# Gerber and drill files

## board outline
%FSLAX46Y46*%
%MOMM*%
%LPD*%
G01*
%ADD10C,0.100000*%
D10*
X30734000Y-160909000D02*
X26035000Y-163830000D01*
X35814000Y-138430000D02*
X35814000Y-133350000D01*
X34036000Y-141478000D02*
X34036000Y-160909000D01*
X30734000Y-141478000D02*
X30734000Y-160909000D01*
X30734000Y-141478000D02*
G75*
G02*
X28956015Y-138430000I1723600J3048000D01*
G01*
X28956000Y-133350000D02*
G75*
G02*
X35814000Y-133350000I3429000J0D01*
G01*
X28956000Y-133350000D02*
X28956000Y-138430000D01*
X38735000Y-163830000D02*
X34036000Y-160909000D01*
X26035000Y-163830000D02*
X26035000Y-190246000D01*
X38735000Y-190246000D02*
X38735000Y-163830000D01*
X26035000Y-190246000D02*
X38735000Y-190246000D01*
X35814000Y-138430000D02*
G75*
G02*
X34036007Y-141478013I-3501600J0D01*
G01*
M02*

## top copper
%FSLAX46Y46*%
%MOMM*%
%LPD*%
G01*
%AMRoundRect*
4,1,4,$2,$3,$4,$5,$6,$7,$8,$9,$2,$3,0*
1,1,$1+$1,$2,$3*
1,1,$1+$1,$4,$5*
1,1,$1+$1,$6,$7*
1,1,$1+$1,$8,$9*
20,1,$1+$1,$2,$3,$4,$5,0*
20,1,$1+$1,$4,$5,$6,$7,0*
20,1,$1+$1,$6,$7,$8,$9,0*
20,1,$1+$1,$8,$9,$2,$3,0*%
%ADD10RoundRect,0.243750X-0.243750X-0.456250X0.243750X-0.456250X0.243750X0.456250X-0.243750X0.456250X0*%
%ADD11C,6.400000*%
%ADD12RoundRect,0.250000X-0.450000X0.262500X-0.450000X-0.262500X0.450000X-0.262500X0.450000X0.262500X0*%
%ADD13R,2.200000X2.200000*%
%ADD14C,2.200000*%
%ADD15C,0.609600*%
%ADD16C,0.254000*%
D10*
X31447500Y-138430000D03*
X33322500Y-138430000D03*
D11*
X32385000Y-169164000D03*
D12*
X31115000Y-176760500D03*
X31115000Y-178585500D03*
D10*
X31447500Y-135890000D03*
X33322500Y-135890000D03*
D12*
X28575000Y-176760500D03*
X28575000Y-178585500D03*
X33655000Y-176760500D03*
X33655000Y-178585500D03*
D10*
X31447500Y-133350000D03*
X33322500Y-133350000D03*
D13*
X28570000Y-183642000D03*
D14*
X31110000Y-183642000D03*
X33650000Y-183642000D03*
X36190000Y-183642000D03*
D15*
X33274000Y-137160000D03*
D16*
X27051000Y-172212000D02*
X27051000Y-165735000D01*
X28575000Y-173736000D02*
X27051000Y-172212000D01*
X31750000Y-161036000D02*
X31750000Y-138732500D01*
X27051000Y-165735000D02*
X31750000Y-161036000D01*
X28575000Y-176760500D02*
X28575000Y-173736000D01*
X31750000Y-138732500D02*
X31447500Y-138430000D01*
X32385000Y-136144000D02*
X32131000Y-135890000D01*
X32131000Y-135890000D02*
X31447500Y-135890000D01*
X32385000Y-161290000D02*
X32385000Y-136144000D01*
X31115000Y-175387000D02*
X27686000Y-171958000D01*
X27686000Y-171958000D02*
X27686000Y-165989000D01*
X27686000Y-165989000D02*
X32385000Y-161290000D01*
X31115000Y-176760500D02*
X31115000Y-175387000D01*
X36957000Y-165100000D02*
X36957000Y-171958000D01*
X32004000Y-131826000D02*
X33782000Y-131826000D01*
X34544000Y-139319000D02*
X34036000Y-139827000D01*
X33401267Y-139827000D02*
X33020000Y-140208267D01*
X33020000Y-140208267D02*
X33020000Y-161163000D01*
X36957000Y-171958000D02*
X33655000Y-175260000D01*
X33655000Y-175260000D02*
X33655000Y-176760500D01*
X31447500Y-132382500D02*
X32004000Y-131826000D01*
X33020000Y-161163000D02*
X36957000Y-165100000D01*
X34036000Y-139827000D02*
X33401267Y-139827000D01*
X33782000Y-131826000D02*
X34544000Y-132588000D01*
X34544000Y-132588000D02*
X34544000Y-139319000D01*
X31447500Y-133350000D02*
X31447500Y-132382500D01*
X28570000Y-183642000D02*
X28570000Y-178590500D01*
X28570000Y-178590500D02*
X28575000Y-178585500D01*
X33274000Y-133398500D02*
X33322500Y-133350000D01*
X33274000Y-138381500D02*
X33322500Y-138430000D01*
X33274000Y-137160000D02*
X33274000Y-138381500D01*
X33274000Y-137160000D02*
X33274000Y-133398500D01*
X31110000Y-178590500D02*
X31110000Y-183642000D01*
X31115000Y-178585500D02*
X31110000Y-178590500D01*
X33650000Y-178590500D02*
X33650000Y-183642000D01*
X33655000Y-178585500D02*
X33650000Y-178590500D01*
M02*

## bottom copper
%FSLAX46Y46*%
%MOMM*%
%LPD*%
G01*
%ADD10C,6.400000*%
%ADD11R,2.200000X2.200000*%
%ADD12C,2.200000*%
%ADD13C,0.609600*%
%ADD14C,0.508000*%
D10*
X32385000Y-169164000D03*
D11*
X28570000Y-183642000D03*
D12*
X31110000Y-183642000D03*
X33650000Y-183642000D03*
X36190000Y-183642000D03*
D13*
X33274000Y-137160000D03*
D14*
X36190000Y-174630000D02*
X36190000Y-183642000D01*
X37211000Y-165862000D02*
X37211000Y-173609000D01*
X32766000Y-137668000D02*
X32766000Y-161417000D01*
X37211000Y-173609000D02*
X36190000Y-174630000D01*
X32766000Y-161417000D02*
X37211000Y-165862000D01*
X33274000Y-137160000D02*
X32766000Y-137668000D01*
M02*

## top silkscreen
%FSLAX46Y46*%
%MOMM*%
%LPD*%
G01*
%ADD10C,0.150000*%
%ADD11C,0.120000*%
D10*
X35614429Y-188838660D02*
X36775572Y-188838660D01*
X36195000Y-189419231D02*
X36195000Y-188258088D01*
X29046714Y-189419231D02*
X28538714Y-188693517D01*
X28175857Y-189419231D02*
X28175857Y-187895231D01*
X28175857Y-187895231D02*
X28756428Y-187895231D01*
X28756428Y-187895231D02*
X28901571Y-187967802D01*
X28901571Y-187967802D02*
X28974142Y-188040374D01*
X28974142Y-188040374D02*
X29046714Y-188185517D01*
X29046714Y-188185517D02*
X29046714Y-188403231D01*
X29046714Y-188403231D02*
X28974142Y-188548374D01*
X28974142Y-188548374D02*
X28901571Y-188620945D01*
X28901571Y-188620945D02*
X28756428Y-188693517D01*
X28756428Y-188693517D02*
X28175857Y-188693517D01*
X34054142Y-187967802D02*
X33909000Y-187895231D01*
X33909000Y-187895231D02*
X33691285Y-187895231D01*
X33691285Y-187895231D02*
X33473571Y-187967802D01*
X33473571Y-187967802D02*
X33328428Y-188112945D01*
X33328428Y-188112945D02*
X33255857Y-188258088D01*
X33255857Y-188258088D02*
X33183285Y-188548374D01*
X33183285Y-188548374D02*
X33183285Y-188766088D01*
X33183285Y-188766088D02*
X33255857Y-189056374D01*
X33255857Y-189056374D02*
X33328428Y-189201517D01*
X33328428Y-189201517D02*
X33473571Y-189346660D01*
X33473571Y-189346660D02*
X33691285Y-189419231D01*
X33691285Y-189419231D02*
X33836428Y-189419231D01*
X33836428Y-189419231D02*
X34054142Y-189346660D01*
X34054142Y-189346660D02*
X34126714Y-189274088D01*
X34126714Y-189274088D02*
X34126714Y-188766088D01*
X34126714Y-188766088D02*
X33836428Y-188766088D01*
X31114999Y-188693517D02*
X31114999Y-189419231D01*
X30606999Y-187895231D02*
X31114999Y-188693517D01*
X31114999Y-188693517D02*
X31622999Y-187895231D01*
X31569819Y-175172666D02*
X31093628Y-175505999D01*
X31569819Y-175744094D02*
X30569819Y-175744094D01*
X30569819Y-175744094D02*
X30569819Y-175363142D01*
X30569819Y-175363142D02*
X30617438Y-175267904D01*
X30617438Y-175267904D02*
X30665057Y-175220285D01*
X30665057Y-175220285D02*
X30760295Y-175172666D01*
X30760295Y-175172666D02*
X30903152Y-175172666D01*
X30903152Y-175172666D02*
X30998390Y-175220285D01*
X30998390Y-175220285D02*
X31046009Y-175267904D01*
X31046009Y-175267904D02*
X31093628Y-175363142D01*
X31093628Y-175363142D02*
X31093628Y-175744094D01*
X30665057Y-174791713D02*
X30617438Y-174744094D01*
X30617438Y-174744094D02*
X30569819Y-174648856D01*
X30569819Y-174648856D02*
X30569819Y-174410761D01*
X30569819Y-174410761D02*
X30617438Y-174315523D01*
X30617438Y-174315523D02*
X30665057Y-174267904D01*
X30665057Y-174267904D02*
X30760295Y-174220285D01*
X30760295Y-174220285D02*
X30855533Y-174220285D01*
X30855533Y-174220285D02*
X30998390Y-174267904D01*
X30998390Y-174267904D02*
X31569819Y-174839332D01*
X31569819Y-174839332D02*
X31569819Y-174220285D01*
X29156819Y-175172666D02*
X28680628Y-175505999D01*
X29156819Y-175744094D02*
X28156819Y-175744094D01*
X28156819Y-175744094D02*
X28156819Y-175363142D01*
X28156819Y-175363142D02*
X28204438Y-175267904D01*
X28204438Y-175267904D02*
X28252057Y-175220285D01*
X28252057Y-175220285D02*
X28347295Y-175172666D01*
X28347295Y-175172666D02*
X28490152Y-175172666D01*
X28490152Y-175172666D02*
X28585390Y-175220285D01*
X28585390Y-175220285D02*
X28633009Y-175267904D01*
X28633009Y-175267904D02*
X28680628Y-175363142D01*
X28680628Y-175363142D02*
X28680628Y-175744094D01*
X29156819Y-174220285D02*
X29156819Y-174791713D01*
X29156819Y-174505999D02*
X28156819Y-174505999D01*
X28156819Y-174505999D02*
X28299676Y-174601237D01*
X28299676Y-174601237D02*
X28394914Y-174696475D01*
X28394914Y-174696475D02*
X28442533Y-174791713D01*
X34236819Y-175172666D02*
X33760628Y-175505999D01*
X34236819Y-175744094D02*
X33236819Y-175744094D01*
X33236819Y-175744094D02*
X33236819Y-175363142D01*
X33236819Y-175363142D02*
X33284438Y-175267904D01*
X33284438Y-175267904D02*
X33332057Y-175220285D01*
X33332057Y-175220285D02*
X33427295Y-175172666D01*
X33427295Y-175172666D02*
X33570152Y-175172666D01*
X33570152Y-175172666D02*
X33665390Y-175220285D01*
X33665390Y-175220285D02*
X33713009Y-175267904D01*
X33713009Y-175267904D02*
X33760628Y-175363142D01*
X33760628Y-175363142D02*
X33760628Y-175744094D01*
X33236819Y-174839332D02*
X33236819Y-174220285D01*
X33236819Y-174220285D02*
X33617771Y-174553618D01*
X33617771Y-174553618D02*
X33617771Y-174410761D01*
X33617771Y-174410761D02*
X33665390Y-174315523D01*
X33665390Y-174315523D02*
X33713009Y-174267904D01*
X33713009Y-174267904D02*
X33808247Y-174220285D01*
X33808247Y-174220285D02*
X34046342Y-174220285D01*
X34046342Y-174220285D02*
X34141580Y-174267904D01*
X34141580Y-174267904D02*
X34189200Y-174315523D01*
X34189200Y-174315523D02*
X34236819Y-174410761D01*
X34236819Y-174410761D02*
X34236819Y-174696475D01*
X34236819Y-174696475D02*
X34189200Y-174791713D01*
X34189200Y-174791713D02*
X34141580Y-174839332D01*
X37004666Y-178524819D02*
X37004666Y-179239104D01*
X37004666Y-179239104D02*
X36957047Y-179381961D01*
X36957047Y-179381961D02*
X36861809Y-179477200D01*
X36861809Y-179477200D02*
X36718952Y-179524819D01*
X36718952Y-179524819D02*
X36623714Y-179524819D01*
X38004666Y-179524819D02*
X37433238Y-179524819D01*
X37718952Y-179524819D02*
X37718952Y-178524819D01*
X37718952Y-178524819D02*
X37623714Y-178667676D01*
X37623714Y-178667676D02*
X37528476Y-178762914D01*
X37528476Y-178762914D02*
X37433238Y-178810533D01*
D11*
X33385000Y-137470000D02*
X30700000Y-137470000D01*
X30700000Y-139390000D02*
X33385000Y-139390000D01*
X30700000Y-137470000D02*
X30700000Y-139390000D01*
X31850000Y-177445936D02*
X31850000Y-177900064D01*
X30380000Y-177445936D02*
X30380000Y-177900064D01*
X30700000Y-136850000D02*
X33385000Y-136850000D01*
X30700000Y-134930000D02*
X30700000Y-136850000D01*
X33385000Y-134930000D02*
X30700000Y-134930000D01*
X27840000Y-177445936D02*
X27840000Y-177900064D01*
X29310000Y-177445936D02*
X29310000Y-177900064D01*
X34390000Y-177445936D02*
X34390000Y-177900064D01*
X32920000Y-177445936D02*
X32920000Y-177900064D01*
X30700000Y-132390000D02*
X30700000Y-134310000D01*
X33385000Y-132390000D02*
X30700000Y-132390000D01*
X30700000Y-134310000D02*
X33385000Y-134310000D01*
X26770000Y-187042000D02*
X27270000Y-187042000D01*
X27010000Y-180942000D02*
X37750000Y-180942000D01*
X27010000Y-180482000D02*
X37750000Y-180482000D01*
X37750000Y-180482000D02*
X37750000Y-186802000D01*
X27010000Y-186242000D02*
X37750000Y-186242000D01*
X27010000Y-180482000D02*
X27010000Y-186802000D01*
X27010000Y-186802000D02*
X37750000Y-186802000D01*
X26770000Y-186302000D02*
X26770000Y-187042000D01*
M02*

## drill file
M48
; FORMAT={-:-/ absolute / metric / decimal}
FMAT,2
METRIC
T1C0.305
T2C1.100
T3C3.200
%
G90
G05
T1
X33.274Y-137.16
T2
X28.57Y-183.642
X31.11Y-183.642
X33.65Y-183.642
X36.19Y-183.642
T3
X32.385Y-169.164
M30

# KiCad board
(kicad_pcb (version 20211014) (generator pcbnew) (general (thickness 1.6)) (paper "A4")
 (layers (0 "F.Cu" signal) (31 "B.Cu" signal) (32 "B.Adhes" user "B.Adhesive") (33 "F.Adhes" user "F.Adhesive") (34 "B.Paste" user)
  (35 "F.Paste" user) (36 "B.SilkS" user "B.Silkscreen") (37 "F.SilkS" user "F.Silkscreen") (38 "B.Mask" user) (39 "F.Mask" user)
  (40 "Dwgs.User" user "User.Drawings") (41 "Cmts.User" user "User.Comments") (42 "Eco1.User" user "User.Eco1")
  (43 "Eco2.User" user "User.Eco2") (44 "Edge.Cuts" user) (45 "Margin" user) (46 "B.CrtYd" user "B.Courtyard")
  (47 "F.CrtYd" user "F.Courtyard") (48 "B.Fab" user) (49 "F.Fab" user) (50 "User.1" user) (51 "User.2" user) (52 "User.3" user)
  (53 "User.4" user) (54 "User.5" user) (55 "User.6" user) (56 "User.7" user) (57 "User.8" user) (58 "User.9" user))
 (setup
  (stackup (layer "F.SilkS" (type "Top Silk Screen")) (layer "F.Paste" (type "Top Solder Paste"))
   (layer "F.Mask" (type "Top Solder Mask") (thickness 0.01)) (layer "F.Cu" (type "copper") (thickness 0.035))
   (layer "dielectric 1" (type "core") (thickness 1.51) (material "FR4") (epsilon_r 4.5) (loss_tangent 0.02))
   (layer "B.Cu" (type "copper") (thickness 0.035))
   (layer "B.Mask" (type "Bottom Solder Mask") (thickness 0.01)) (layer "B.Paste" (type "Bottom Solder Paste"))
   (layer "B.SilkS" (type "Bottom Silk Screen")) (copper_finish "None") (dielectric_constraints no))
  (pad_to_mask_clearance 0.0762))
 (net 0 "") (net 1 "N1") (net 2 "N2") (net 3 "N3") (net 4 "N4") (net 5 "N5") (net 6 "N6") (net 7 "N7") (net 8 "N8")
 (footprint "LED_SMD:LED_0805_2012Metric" (layer "F.Cu") (at 32.385 138.43)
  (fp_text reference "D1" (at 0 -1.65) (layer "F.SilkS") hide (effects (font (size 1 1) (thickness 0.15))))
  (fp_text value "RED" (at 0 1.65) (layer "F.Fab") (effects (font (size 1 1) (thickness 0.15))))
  (fp_line (start 1 -0.96) (end -1.685 -0.96) (layer "F.SilkS") (width 0.12))
  (fp_line (start -1.685 0.96) (end 1 0.96) (layer "F.SilkS") (width 0.12))
  (fp_line (start -1.685 -0.96) (end -1.685 0.96) (layer "F.SilkS") (width 0.12))
  (pad "1" smd roundrect (at -0.9375 0) (size 0.975 1.4) (layers "F.Cu" "F.Paste" "F.Mask") (roundrect_rratio 0.25) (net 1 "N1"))
  (pad "2" smd roundrect (at 0.9375 0) (size 0.975 1.4) (layers "F.Cu" "F.Paste" "F.Mask") (roundrect_rratio 0.25) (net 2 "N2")))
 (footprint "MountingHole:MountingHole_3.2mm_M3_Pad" (layer "F.Cu") (at 32.385 169.164) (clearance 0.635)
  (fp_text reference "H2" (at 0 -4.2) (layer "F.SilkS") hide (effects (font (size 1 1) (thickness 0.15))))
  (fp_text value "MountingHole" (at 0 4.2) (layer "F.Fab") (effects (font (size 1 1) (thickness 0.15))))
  (pad "1" thru_hole circle (at 0 0) (size 6.4 6.4) (drill 3.2) (layers *.Cu *.Mask) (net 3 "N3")))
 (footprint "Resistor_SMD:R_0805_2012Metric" (layer "F.Cu") (at 31.115 177.673 -90)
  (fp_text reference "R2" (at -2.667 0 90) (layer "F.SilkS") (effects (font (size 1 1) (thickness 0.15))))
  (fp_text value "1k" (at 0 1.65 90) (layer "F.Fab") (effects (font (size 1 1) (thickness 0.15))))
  (fp_line (start -0.227064 -0.735) (end 0.227064 -0.735) (layer "F.SilkS") (width 0.12))
  (fp_line (start -0.227064 0.735) (end 0.227064 0.735) (layer "F.SilkS") (width 0.12))
  (pad "1" smd roundrect (at -0.9125 0 270) (size 1.025 1.4) (layers "F.Cu" "F.Paste" "F.Mask") (roundrect_rratio 0.243902) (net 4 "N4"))
  (pad "2" smd roundrect (at 0.9125 0 270) (size 1.025 1.4) (layers "F.Cu" "F.Paste" "F.Mask") (roundrect_rratio 0.243902) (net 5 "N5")))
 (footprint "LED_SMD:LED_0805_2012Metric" (layer "F.Cu") (at 32.385 135.89)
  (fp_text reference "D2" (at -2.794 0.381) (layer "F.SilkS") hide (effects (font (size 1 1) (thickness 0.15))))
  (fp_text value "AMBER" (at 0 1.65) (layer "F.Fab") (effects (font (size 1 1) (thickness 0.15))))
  (fp_line (start -1.685 0.96) (end 1 0.96) (layer "F.SilkS") (width 0.12))
  (fp_line (start -1.685 -0.96) (end -1.685 0.96) (layer "F.SilkS") (width 0.12))
  (fp_line (start 1 -0.96) (end -1.685 -0.96) (layer "F.SilkS") (width 0.12))
  (pad "1" smd roundrect (at -0.9375 0) (size 0.975 1.4) (layers "F.Cu" "F.Paste" "F.Mask") (roundrect_rratio 0.25) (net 4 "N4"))
  (pad "2" smd roundrect (at 0.9375 0) (size 0.975 1.4) (layers "F.Cu" "F.Paste" "F.Mask") (roundrect_rratio 0.25) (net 2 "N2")))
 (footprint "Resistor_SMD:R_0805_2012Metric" (layer "F.Cu") (at 28.575 177.673 -90)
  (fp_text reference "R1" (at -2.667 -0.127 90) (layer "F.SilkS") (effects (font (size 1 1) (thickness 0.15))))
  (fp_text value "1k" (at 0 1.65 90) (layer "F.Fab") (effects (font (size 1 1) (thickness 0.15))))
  (fp_line (start -0.227064 0.735) (end 0.227064 0.735) (layer "F.SilkS") (width 0.12))
  (fp_line (start -0.227064 -0.735) (end 0.227064 -0.735) (layer "F.SilkS") (width 0.12))
  (pad "1" smd roundrect (at -0.9125 0 270) (size 1.025 1.4) (layers "F.Cu" "F.Paste" "F.Mask") (roundrect_rratio 0.243902) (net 1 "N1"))
  (pad "2" smd roundrect (at 0.9125 0 270) (size 1.025 1.4) (layers "F.Cu" "F.Paste" "F.Mask") (roundrect_rratio 0.243902) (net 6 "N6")))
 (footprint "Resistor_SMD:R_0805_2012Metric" (layer "F.Cu") (at 33.655 177.673 -90)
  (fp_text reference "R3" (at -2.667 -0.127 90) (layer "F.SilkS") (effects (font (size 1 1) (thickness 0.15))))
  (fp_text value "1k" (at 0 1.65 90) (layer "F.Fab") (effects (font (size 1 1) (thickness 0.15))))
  (fp_line (start -0.227064 -0.735) (end 0.227064 -0.735) (layer "F.SilkS") (width 0.12))
  (fp_line (start -0.227064 0.735) (end 0.227064 0.735) (layer "F.SilkS") (width 0.12))
  (pad "1" smd roundrect (at -0.9125 0 270) (size 1.025 1.4) (layers "F.Cu" "F.Paste" "F.Mask") (roundrect_rratio 0.243902) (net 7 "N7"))
  (pad "2" smd roundrect (at 0.9125 0 270) (size 1.025 1.4) (layers "F.Cu" "F.Paste" "F.Mask") (roundrect_rratio 0.243902) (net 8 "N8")))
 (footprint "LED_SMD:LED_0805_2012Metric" (layer "F.Cu") (at 32.385 133.35)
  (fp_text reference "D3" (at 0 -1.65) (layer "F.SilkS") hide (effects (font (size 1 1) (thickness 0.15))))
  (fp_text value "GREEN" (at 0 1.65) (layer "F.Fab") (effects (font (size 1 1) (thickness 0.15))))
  (fp_line (start -1.685 -0.96) (end -1.685 0.96) (layer "F.SilkS") (width 0.12))
  (fp_line (start 1 -0.96) (end -1.685 -0.96) (layer "F.SilkS") (width 0.12))
  (fp_line (start -1.685 0.96) (end 1 0.96) (layer "F.SilkS") (width 0.12))
  (pad "1" smd roundrect (at -0.9375 0) (size 0.975 1.4) (layers "F.Cu" "F.Paste" "F.Mask") (roundrect_rratio 0.25) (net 7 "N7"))
  (pad "2" smd roundrect (at 0.9375 0) (size 0.975 1.4) (layers "F.Cu" "F.Paste" "F.Mask") (roundrect_rratio 0.25) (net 2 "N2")))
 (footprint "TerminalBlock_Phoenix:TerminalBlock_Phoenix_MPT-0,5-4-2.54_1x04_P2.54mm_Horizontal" (layer "F.Cu") (at 28.57 183.642)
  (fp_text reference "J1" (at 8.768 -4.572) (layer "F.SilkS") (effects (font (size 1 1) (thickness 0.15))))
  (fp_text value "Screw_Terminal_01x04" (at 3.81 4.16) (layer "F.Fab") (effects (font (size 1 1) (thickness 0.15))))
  (fp_line (start -1.8 3.4) (end -1.3 3.4) (layer "F.SilkS") (width 0.12))
  (fp_line (start -1.56 -2.7) (end 9.18 -2.7) (layer "F.SilkS") (width 0.12))
  (fp_line (start -1.56 -3.16) (end 9.18 -3.16) (layer "F.SilkS") (width 0.12))
  (fp_line (start 9.18 -3.16) (end 9.18 3.16) (layer "F.SilkS") (width 0.12))
  (fp_line (start -1.56 2.6) (end 9.18 2.6) (layer "F.SilkS") (width 0.12))
  (fp_line (start -1.56 -3.16) (end -1.56 3.16) (layer "F.SilkS") (width 0.12))
  (fp_line (start -1.56 3.16) (end 9.18 3.16) (layer "F.SilkS") (width 0.12))
  (fp_line (start -1.8 2.66) (end -1.8 3.4) (layer "F.SilkS") (width 0.12))
  (pad "1" thru_hole rect (at 0 0) (size 2.2 2.2) (drill 1.1) (layers *.Cu *.Mask) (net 6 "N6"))
  (pad "2" thru_hole circle (at 2.54 0) (size 2.2 2.2) (drill 1.1) (layers *.Cu *.Mask) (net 5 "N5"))
  (pad "3" thru_hole circle (at 5.08 0) (size 2.2 2.2) (drill 1.1) (layers *.Cu *.Mask) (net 8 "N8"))
  (pad "4" thru_hole circle (at 7.62 0) (size 2.2 2.2) (drill 1.1) (layers *.Cu *.Mask) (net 2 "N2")))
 (gr_line (start 30.734 160.909) (end 26.035 163.83) (layer "Edge.Cuts") (width 0.1))
 (gr_line (start 35.814 138.43) (end 35.814 133.35) (layer "Edge.Cuts") (width 0.1))
 (gr_line (start 34.036 141.478) (end 34.036 160.909) (layer "Edge.Cuts") (width 0.1))
 (gr_line (start 30.734 141.478) (end 30.734 160.909) (layer "Edge.Cuts") (width 0.1))
 (gr_arc (start 30.734 141.478) (mid 29.432988 140.19434) (end 28.956 138.43) (layer "Edge.Cuts") (width 0.1))
 (gr_arc (start 28.956 133.35) (mid 32.385 129.921) (end 35.814 133.35) (layer "Edge.Cuts") (width 0.1))
 (gr_line (start 28.956 133.35) (end 28.956 138.43) (layer "Edge.Cuts") (width 0.1))
 (gr_line (start 38.735 163.83) (end 34.036 160.909) (layer "Edge.Cuts") (width 0.1))
 (gr_line (start 26.035 163.83) (end 26.035 190.246) (layer "Edge.Cuts") (width 0.1))
 (gr_line (start 38.735 190.246) (end 38.735 163.83) (layer "Edge.Cuts") (width 0.1))
 (gr_line (start 26.035 190.246) (end 38.735 190.246) (layer "Edge.Cuts") (width 0.1))
 (gr_arc (start 35.814 138.43) (mid 35.337012 140.19434) (end 34.036 141.478) (layer "Edge.Cuts") (width 0.1))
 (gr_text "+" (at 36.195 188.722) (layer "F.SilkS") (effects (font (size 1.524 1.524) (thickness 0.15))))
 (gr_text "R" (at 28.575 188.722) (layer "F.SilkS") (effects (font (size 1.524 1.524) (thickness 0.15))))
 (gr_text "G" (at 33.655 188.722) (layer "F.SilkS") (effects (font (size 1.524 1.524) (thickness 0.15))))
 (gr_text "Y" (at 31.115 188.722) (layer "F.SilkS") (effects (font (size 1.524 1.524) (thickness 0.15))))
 (segment (start 27.051 172.212) (end 27.051 165.735) (width 0.254) (layer "F.Cu") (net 1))
 (segment (start 28.575 173.736) (end 27.051 172.212) (width 0.254) (layer "F.Cu") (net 1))
 (segment (start 31.75 161.036) (end 31.75 138.7325) (width 0.254) (layer "F.Cu") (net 1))
 (segment (start 27.051 165.735) (end 31.75 161.036) (width 0.254) (layer "F.Cu") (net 1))
 (segment (start 28.575 176.7605) (end 28.575 173.736) (width 0.254) (layer "F.Cu") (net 1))
 (segment (start 31.75 138.7325) (end 31.4475 138.43) (width 0.254) (layer "F.Cu") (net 1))
 (segment (start 32.385 136.144) (end 32.131 135.89) (width 0.254) (layer "F.Cu") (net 4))
 (segment (start 32.131 135.89) (end 31.4475 135.89) (width 0.254) (layer "F.Cu") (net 4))
 (segment (start 32.385 161.29) (end 32.385 136.144) (width 0.254) (layer "F.Cu") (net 4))
 (segment (start 31.115 175.387) (end 27.686 171.958) (width 0.254) (layer "F.Cu") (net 4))
 (segment (start 27.686 171.958) (end 27.686 165.989) (width 0.254) (layer "F.Cu") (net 4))
 (segment (start 27.686 165.989) (end 32.385 161.29) (width 0.254) (layer "F.Cu") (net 4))
 (segment (start 31.115 176.7605) (end 31.115 175.387) (width 0.254) (layer "F.Cu") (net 4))
 (segment (start 36.957 165.1) (end 36.957 171.958) (width 0.254) (layer "F.Cu") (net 7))
 (segment (start 32.004 131.826) (end 33.782 131.826) (width 0.254) (layer "F.Cu") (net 7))
 (segment (start 34.544 139.319) (end 34.036 139.827) (width 0.254) (layer "F.Cu") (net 7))
 (segment (start 33.401267 139.827) (end 33.02 140.208267) (width 0.254) (layer "F.Cu") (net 7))
 (segment (start 33.02 140.208267) (end 33.02 161.163) (width 0.254) (layer "F.Cu") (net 7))
 (segment (start 36.957 171.958) (end 33.655 175.26) (width 0.254) (layer "F.Cu") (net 7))
 (segment (start 33.655 175.26) (end 33.655 176.7605) (width 0.254) (layer "F.Cu") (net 7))
 (segment (start 31.4475 132.3825) (end 32.004 131.826) (width 0.254) (layer "F.Cu") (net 7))
 (segment (start 33.02 161.163) (end 36.957 165.1) (width 0.254) (layer "F.Cu") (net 7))
 (segment (start 34.036 139.827) (end 33.401267 139.827) (width 0.254) (layer "F.Cu") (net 7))
 (segment (start 33.782 131.826) (end 34.544 132.588) (width 0.254) (layer "F.Cu") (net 7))
 (segment (start 34.544 132.588) (end 34.544 139.319) (width 0.254) (layer "F.Cu") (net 7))
 (segment (start 31.4475 133.35) (end 31.4475 132.3825) (width 0.254) (layer "F.Cu") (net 7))
 (segment (start 28.57 183.642) (end 28.57 178.5905) (width 0.254) (layer "F.Cu") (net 6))
 (segment (start 28.57 178.5905) (end 28.575 178.5855) (width 0.254) (layer "F.Cu") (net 6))
 (segment (start 33.274 133.3985) (end 33.3225 133.35) (width 0.254) (layer "F.Cu") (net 2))
 (segment (start 33.274 138.3815) (end 33.3225 138.43) (width 0.254) (layer "F.Cu") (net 2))
 (segment (start 33.274 137.16) (end 33.274 138.3815) (width 0.254) (layer "F.Cu") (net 2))
 (segment (start 33.274 137.16) (end 33.274 133.3985) (width 0.254) (layer "F.Cu") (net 2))
 (via (at 33.274 137.16) (size 0.6096) (drill 0.3048) (layers "F.Cu" "B.Cu") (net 2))
 (segment (start 36.19 174.63) (end 36.19 183.642) (width 0.508) (layer "B.Cu") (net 2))
 (segment (start 37.211 165.862) (end 37.211 173.609) (width 0.508) (layer "B.Cu") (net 2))
 (segment (start 32.766 137.668) (end 32.766 161.417) (width 0.508) (layer "B.Cu") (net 2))
 (segment (start 37.211 173.609) (end 36.19 174.63) (width 0.508) (layer "B.Cu") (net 2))
 (segment (start 32.766 161.417) (end 37.211 165.862) (width 0.508) (layer "B.Cu") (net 2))
 (segment (start 33.274 137.16) (end 32.766 137.668) (width 0.508) (layer "B.Cu") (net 2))
 (segment (start 31.11 178.5905) (end 31.11 183.642) (width 0.254) (layer "F.Cu") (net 5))
 (segment (start 31.115 178.5855) (end 31.11 178.5905) (width 0.254) (layer "F.Cu") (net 5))
 (segment (start 33.65 178.5905) (end 33.65 183.642) (width 0.254) (layer "F.Cu") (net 8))
 (segment (start 33.655 178.5855) (end 33.65 178.5905) (width 0.254) (layer "F.Cu") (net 8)))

